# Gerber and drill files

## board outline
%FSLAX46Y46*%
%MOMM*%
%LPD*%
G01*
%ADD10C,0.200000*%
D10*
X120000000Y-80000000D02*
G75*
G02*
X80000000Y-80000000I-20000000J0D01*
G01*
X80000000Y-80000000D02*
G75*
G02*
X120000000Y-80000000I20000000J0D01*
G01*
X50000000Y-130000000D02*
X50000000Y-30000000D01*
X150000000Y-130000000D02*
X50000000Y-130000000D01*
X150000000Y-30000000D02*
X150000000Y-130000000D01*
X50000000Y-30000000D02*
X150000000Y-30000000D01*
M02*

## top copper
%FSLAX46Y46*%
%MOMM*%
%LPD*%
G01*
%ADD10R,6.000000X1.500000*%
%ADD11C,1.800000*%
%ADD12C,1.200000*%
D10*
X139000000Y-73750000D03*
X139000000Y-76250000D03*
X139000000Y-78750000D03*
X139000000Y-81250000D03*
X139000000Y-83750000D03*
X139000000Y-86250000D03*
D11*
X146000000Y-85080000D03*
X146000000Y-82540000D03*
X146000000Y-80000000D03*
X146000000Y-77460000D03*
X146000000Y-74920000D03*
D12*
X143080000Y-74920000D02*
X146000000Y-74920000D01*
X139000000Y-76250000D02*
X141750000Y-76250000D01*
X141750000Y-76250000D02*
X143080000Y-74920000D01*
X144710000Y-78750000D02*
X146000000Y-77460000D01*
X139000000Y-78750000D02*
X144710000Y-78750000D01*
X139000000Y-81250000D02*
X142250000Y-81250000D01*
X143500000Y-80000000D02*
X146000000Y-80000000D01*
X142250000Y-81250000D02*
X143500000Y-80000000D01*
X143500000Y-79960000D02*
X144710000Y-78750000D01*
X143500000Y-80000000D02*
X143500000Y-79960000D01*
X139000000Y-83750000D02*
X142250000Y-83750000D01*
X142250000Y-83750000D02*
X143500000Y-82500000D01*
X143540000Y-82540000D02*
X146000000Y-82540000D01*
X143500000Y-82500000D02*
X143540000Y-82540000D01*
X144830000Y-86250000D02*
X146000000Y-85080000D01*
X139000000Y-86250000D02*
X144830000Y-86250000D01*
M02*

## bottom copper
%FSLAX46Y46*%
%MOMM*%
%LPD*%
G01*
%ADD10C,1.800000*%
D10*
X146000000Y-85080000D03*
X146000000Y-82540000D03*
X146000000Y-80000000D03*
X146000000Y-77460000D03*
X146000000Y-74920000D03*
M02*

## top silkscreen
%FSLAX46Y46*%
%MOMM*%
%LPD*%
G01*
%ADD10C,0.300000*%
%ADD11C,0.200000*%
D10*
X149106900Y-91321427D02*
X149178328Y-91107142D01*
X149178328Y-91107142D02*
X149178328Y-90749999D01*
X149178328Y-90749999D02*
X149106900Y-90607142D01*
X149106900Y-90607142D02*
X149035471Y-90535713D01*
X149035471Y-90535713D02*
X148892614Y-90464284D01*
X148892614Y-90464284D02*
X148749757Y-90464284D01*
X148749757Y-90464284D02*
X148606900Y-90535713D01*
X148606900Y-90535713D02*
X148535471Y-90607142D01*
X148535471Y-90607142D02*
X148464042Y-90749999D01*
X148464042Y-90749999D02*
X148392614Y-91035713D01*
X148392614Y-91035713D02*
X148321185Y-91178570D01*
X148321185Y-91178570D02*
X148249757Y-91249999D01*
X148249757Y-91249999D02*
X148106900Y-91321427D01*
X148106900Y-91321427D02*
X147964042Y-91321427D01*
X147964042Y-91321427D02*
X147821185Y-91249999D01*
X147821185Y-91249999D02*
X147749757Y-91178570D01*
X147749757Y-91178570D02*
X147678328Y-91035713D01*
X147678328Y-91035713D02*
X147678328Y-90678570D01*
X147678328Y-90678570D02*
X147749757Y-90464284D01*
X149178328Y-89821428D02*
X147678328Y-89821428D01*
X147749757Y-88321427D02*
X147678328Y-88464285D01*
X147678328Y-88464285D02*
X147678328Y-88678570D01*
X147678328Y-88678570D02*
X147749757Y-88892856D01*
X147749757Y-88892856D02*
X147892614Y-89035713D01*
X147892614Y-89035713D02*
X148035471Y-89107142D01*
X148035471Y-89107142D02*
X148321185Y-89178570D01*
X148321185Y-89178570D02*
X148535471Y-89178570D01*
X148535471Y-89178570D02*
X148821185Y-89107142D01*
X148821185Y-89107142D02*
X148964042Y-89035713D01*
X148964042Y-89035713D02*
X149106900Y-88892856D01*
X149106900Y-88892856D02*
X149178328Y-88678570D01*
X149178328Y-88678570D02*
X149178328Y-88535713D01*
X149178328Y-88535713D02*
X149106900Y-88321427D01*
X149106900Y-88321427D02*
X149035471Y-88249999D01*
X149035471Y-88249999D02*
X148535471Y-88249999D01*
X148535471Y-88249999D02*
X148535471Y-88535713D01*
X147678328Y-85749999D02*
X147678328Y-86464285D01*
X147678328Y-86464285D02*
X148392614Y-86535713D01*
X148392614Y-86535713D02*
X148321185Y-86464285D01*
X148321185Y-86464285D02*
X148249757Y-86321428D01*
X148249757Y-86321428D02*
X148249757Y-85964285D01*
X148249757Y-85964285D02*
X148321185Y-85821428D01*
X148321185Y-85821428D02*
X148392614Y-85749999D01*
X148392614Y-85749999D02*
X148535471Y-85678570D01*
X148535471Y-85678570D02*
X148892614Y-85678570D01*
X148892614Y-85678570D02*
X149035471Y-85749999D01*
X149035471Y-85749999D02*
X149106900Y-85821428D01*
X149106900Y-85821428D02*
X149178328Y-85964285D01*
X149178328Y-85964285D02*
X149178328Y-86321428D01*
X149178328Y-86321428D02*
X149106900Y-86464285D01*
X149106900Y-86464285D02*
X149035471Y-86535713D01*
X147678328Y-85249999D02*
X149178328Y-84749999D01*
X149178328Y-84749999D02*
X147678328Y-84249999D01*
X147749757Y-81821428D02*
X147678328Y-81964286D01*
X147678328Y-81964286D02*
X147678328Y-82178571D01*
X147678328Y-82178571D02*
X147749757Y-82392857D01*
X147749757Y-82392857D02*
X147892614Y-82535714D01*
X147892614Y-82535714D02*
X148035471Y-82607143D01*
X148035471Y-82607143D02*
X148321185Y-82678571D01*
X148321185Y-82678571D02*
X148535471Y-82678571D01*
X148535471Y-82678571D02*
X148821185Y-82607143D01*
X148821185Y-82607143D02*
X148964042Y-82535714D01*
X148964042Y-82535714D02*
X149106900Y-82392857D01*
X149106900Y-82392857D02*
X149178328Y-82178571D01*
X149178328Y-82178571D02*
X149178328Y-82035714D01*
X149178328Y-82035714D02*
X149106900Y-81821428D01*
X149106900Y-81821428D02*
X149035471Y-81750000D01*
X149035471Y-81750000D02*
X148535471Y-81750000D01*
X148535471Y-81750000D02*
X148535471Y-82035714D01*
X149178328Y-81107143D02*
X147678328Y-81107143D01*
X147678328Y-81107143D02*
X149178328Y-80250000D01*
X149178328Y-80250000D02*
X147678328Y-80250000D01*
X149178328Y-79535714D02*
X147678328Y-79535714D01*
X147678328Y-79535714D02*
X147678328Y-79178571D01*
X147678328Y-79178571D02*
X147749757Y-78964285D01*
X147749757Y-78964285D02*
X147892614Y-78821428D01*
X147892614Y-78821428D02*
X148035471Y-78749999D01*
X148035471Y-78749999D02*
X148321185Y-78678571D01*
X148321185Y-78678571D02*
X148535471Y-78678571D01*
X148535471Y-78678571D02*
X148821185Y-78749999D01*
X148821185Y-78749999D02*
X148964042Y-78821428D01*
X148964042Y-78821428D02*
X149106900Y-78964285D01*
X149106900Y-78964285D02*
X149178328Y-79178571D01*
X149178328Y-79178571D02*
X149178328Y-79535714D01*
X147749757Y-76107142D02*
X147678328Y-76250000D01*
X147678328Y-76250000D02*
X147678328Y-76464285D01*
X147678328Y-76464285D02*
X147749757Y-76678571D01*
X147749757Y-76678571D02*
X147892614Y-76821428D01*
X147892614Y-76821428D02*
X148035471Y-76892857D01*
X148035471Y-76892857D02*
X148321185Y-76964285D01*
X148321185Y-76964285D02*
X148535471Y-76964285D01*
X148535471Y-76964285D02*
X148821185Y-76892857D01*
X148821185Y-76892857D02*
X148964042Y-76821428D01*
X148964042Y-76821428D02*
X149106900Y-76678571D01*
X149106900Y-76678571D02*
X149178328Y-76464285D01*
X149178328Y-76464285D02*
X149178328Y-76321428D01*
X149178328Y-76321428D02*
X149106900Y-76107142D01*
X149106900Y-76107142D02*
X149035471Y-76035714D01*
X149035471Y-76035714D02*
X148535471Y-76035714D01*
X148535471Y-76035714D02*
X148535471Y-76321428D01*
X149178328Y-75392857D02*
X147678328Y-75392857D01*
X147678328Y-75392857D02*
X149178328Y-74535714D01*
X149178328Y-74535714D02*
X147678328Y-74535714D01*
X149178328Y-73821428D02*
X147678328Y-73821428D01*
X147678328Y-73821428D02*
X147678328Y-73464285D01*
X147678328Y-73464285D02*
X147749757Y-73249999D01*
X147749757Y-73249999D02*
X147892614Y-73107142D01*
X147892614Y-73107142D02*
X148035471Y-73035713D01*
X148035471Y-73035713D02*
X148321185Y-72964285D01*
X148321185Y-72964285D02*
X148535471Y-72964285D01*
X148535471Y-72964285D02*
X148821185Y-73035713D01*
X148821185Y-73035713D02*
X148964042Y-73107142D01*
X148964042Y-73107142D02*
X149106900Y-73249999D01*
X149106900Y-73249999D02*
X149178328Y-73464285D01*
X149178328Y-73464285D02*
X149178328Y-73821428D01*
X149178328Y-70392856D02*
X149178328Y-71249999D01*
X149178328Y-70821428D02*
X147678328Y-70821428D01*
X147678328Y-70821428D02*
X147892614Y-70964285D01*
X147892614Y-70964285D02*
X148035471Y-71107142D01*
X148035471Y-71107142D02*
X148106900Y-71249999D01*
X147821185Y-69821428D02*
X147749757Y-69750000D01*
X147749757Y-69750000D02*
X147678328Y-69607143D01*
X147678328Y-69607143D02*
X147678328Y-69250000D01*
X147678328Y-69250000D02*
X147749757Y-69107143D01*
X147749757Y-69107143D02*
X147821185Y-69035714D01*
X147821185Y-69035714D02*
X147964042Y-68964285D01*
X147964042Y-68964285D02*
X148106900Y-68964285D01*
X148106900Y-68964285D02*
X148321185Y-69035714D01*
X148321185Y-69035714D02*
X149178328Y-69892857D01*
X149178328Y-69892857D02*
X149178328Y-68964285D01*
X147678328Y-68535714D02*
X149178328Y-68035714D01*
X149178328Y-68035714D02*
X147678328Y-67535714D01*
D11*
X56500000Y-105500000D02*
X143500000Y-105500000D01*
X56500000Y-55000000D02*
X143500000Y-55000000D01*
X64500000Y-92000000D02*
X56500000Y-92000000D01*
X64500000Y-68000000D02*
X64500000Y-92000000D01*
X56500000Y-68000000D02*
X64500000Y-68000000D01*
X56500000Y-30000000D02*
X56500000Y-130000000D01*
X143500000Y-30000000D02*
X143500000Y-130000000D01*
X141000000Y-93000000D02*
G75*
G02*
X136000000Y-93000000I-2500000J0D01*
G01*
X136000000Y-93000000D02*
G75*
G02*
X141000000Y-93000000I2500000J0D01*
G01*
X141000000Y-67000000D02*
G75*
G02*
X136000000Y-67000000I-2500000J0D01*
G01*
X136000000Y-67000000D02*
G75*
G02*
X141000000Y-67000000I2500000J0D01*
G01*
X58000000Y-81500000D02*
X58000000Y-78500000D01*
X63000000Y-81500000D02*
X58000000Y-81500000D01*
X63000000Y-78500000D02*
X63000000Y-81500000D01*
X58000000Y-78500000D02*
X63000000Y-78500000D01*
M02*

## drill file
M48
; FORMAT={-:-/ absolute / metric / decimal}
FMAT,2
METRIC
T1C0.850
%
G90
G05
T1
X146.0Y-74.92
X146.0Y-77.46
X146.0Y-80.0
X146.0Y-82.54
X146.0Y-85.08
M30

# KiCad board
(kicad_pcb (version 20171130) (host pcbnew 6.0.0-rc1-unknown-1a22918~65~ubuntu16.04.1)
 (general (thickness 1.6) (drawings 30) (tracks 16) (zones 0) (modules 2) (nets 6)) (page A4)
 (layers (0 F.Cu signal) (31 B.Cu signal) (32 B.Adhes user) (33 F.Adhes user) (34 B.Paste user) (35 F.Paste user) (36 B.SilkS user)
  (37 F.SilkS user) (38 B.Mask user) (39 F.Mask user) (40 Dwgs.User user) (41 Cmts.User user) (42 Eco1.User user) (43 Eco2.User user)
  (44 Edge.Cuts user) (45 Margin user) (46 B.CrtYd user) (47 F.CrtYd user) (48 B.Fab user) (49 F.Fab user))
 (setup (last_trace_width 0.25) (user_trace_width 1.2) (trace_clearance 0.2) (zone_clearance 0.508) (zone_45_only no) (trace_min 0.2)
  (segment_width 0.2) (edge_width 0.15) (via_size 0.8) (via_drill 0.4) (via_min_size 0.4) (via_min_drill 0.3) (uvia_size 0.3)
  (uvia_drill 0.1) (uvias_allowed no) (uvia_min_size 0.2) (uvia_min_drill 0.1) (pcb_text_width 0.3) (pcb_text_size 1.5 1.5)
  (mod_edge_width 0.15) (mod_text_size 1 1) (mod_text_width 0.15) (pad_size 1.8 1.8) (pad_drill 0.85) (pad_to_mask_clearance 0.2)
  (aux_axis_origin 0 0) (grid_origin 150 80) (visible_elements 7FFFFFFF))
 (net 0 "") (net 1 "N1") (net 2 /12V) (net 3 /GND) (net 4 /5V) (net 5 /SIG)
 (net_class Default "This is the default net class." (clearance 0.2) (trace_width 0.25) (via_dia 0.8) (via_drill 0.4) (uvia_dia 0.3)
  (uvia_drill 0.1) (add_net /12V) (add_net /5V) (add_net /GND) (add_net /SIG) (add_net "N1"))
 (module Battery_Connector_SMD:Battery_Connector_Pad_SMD (layer F.Cu) (at 139 80 270)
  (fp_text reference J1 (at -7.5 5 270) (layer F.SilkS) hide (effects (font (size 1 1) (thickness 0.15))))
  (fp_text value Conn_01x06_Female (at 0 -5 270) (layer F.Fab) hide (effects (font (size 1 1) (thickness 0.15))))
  (pad 1 smd rect (at -6.25 0 270) (size 1.5 6) (layers F.Cu F.Mask) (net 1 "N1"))
  (pad 2 smd rect (at -3.75 0 270) (size 1.5 6) (layers F.Cu F.Mask) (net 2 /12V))
  (pad 3 smd rect (at -1.25 0 270) (size 1.5 6) (layers F.Cu F.Mask) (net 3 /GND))
  (pad 4 smd rect (at 1.25 0 270) (size 1.5 6) (layers F.Cu F.Mask) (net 3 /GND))
  (pad 5 smd rect (at 3.75 0 270) (size 1.5 6) (layers F.Cu F.Mask) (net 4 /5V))
  (pad 6 smd rect (at 6.25 0 270) (size 1.5 6) (layers F.Cu F.Mask) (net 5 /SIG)))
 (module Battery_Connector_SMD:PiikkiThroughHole (layer F.Cu) (at 146 80 270)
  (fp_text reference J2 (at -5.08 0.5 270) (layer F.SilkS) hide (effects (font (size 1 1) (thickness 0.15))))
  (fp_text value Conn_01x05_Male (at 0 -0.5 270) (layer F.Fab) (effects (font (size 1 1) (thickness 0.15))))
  (pad 5 thru_hole circle (at 5.08 0 270) (size 1.8 1.8) (drill 0.85) (layers *.Cu *.Mask) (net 5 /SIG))
  (pad 4 thru_hole circle (at 2.54 0 270) (size 1.8 1.8) (drill 0.85) (layers *.Cu *.Mask) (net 4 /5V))
  (pad 3 thru_hole circle (at 0 0 270) (size 1.8 1.8) (drill 0.85) (layers *.Cu *.Mask) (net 3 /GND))
  (pad 2 thru_hole circle (at -2.54 0 270) (size 1.8 1.8) (drill 0.85) (layers *.Cu *.Mask) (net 3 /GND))
  (pad 1 thru_hole circle (at -5.08 0 270) (size 1.8 1.8) (drill 0.85) (layers *.Cu *.Mask) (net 2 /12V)))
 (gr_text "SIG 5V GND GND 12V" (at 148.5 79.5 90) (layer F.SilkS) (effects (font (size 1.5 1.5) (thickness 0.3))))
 (gr_circle (center 100 80) (end 80 80) (layer Edge.Cuts) (width 0.2))
 (gr_line (start 56.5 105.5) (end 143.5 105.5) (layer F.SilkS) (width 0.2))
 (gr_line (start 56.5 55) (end 143.5 55) (layer F.SilkS) (width 0.2))
 (gr_line (start 64.5 92) (end 56.5 92) (layer F.SilkS) (width 0.2))
 (gr_line (start 64.5 68) (end 64.5 92) (layer F.SilkS) (width 0.2))
 (gr_line (start 56.5 68) (end 64.5 68) (layer F.SilkS) (width 0.2))
 (gr_line (start 56.5 30) (end 56.5 130) (layer F.SilkS) (width 0.2))
 (gr_line (start 143.5 30) (end 143.5 130) (layer F.SilkS) (width 0.2))
 (gr_circle (center 138.5 93) (end 141 93) (layer F.SilkS) (width 0.2))
 (gr_circle (center 138.5 67) (end 141 67) (layer F.SilkS) (width 0.2))
 (gr_line (start 58 81.5) (end 58 78.5) (layer F.SilkS) (width 0.2))
 (gr_line (start 63 81.5) (end 58 81.5) (layer F.SilkS) (width 0.2))
 (gr_line (start 63 78.5) (end 63 81.5) (layer F.SilkS) (width 0.2))
 (gr_line (start 58 78.5) (end 63 78.5) (layer F.SilkS) (width 0.2))
 (gr_line (start 50 130) (end 50 30) (layer Edge.Cuts) (width 0.2))
 (gr_line (start 150 130) (end 50 130) (layer Edge.Cuts) (width 0.2))
 (gr_line (start 150 30) (end 150 130) (layer Edge.Cuts) (width 0.2))
 (gr_line (start 50 30) (end 150 30) (layer Edge.Cuts) (width 0.2))
 (segment (start 143.08 74.92) (end 146 74.92) (width 1.2) (layer F.Cu) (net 2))
 (segment (start 139 76.25) (end 141.75 76.25) (width 1.2) (layer F.Cu) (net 2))
 (segment (start 141.75 76.25) (end 143.08 74.92) (width 1.2) (layer F.Cu) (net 2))
 (segment (start 144.71 78.75) (end 146 77.46) (width 1.2) (layer F.Cu) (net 3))
 (segment (start 139 78.75) (end 144.71 78.75) (width 1.2) (layer F.Cu) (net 3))
 (segment (start 139 81.25) (end 142.25 81.25) (width 1.2) (layer F.Cu) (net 3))
 (segment (start 143.5 80) (end 146 80) (width 1.2) (layer F.Cu) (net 3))
 (segment (start 142.25 81.25) (end 143.5 80) (width 1.2) (layer F.Cu) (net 3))
 (segment (start 143.5 79.96) (end 144.71 78.75) (width 1.2) (layer F.Cu) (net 3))
 (segment (start 143.5 80) (end 143.5 79.96) (width 1.2) (layer F.Cu) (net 3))
 (segment (start 139 83.75) (end 142.25 83.75) (width 1.2) (layer F.Cu) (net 4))
 (segment (start 142.25 83.75) (end 143.5 82.5) (width 1.2) (layer F.Cu) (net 4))
 (segment (start 143.54 82.54) (end 146 82.54) (width 1.2) (layer F.Cu) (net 4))
 (segment (start 143.5 82.5) (end 143.54 82.54) (width 1.2) (layer F.Cu) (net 4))
 (segment (start 144.83 86.25) (end 146 85.08) (width 1.2) (layer F.Cu) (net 5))
 (segment (start 139 86.25) (end 144.83 86.25) (width 1.2) (layer F.Cu) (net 5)))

